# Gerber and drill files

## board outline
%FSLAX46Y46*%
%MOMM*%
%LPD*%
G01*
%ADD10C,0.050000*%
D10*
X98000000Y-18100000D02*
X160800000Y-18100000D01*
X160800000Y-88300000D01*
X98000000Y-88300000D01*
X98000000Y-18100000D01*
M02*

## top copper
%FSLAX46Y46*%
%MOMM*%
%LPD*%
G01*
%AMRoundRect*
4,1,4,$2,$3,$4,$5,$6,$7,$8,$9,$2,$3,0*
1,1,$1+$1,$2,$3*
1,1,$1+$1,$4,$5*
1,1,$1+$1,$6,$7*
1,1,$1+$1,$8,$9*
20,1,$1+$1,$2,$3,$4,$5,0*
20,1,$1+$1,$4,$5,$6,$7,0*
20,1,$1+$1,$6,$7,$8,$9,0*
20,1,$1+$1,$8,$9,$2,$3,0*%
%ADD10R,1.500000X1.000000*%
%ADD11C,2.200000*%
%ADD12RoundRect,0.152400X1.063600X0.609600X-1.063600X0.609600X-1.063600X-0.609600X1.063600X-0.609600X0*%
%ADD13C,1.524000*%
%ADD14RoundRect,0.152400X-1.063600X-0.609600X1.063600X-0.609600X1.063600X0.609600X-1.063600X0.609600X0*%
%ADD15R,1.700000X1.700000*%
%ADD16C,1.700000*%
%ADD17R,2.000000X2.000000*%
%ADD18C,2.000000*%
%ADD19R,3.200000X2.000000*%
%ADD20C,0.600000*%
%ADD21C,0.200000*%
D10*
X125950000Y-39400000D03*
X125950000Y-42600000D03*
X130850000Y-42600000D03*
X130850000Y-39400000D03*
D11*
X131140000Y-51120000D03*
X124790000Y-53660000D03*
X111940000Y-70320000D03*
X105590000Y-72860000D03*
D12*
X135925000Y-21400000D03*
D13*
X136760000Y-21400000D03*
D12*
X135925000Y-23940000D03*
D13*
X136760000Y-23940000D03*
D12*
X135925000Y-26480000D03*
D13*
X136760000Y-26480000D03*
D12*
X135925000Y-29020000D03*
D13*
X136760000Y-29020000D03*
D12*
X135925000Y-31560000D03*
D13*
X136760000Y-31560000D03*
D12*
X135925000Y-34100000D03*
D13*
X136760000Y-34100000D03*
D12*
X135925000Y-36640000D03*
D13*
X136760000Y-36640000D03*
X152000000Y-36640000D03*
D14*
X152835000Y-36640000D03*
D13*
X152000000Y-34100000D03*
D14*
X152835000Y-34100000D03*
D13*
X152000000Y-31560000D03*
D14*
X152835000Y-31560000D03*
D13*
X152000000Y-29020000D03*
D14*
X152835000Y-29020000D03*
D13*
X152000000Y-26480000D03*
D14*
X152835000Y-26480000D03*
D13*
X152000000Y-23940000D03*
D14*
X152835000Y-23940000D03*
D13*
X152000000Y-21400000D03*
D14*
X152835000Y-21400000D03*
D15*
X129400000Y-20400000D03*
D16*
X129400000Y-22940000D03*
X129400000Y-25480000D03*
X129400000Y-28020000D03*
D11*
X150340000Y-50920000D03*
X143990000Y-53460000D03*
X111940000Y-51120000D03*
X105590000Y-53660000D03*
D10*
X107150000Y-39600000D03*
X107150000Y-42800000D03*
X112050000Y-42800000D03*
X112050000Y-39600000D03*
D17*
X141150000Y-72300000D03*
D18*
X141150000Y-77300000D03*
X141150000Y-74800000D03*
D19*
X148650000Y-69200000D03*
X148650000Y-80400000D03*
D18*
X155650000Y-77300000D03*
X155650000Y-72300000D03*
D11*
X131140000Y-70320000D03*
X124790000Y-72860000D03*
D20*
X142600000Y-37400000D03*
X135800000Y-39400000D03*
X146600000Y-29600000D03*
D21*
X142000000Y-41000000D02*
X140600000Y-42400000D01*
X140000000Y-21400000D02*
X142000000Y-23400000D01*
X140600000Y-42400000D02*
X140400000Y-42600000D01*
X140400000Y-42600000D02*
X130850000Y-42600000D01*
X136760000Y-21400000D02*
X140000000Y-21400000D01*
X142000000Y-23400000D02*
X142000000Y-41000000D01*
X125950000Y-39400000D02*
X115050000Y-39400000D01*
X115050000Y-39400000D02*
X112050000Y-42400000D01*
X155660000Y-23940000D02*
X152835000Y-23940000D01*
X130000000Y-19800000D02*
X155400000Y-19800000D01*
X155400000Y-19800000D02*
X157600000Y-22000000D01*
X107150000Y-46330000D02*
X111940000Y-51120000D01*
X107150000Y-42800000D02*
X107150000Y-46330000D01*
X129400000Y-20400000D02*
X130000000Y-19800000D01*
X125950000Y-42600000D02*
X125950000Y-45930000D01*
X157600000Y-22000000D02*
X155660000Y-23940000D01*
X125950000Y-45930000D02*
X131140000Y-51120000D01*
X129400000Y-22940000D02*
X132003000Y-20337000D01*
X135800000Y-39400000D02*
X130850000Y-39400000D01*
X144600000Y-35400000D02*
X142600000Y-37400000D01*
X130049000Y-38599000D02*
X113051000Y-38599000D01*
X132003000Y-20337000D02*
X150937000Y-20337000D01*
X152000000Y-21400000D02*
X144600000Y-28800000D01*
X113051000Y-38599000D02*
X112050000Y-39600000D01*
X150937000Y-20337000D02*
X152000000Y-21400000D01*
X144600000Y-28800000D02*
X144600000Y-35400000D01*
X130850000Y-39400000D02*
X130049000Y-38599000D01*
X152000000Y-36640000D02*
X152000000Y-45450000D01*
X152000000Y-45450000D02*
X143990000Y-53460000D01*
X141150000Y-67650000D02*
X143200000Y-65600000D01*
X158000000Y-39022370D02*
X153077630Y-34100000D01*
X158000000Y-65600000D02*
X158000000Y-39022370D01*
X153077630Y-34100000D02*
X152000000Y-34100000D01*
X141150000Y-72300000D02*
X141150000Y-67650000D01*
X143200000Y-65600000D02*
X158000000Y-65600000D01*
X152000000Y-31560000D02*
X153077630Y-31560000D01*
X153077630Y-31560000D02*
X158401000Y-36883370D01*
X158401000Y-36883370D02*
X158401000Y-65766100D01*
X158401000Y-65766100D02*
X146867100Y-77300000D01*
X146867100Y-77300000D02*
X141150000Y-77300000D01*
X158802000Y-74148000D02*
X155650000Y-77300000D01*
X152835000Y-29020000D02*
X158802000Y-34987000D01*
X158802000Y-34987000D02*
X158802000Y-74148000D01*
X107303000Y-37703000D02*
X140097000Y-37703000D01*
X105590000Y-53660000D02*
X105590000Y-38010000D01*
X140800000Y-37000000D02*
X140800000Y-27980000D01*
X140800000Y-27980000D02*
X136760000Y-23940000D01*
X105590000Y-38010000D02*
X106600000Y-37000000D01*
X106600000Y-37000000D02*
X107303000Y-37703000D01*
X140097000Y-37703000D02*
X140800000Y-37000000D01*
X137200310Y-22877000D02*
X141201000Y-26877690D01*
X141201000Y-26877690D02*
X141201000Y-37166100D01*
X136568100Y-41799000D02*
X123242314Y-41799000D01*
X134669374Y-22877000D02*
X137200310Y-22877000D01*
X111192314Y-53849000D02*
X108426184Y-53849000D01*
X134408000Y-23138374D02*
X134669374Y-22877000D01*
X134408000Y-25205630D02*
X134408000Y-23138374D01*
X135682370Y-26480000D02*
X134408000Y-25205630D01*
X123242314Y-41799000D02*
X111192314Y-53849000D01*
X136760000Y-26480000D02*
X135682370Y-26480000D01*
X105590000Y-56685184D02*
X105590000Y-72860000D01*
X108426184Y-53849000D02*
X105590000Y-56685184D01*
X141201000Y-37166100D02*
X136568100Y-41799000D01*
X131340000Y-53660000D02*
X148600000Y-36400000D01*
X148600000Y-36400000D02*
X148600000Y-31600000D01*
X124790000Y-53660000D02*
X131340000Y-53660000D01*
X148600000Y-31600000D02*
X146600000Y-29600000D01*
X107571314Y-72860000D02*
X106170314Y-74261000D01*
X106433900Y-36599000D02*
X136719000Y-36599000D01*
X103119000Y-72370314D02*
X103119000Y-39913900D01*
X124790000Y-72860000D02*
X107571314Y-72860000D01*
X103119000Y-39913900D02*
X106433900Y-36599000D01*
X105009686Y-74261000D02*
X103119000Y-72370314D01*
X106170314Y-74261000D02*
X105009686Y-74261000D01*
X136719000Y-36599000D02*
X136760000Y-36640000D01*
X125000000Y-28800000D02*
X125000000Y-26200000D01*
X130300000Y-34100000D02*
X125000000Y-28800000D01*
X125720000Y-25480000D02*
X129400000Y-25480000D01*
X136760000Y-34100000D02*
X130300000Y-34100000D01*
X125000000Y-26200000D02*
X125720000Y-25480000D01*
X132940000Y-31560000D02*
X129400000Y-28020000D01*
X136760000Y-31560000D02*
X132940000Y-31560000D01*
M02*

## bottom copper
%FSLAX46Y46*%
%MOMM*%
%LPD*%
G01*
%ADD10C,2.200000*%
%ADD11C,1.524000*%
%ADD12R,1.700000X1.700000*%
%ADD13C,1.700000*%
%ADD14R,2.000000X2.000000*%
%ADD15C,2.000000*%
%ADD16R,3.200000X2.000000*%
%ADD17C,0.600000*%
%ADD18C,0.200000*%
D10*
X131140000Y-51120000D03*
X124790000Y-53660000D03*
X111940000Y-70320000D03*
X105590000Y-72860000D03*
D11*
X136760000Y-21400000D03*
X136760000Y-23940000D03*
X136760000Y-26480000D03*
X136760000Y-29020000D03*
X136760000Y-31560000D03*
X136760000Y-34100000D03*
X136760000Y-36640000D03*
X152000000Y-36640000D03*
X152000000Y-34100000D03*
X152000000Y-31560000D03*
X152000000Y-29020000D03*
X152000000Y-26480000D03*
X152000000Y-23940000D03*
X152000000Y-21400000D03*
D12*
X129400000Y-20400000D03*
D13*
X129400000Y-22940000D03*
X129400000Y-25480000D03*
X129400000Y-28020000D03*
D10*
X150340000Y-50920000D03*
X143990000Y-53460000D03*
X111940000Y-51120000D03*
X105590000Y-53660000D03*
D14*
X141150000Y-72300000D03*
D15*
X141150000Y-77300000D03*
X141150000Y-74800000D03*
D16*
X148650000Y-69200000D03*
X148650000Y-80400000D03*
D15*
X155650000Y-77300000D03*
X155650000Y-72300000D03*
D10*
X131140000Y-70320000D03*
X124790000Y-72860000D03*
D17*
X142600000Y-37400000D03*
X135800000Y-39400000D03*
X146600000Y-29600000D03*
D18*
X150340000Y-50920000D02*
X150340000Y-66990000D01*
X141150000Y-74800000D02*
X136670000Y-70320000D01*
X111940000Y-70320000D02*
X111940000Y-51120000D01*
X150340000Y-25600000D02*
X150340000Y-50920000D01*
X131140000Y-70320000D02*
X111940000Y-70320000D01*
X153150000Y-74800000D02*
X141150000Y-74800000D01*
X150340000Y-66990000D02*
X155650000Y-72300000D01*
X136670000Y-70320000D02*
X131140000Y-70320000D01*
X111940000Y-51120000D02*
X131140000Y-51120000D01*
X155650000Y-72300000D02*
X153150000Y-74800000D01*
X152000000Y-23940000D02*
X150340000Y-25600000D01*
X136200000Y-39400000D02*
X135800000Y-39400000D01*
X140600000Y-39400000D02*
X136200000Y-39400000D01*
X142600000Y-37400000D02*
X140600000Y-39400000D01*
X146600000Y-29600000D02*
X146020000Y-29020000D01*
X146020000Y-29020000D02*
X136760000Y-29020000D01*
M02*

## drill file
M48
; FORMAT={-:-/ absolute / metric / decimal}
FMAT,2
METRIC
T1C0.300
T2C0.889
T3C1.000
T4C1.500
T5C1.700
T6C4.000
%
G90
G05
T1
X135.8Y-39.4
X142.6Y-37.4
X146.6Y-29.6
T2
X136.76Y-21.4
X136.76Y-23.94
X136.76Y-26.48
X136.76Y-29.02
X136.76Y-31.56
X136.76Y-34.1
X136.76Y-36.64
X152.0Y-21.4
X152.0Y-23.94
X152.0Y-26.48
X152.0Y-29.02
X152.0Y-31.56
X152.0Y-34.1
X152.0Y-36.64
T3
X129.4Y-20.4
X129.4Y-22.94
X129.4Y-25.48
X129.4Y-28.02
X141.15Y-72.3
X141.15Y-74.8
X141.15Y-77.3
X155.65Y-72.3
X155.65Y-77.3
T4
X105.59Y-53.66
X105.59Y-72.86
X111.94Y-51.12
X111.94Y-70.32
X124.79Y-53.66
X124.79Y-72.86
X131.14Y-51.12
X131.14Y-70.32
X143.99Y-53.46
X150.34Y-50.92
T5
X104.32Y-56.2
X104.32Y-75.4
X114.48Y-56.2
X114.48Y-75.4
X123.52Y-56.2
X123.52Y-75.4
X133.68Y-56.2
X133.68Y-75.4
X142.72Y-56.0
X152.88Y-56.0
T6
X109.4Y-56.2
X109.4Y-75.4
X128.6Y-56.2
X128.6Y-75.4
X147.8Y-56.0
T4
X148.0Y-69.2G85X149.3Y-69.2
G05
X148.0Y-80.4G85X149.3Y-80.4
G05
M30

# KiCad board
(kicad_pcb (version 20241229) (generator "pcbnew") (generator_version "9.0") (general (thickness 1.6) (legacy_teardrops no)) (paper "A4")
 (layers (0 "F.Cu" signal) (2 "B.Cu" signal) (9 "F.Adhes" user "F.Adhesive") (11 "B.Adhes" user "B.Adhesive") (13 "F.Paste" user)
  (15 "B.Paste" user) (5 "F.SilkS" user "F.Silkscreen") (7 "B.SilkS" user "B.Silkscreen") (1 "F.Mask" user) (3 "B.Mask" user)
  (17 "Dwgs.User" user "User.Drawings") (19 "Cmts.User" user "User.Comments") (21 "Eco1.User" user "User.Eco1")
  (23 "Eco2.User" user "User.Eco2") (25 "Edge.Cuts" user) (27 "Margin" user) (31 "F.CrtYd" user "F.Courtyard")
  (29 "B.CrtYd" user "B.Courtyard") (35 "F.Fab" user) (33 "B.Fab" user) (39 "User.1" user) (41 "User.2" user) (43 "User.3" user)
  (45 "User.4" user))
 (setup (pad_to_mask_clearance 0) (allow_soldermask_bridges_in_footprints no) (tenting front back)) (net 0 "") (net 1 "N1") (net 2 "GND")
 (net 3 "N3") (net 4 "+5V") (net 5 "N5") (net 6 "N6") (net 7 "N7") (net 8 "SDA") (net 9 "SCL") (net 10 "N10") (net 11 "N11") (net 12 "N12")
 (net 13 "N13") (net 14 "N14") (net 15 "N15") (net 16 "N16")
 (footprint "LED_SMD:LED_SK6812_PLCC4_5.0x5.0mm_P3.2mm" (layer "F.Cu") (at 128.4 41)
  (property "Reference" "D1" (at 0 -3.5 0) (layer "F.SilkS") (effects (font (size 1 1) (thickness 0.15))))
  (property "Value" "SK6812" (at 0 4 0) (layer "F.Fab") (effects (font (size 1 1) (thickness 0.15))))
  (pad "1" smd rect (at -2.45 -1.6 180) (size 1.5 1) (layers "F.Cu" "F.Mask" "F.Paste") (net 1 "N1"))
  (pad "2" smd rect (at -2.45 1.6 180) (size 1.5 1) (layers "F.Cu" "F.Mask" "F.Paste") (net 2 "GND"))
  (pad "3" smd rect (at 2.45 1.6 180) (size 1.5 1) (layers "F.Cu" "F.Mask" "F.Paste") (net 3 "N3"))
  (pad "4" smd rect (at 2.45 -1.6 180) (size 1.5 1) (layers "F.Cu" "F.Mask" "F.Paste") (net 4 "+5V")))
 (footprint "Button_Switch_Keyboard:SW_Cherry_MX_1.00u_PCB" (layer "F.Cu") (at 131.14 51.12)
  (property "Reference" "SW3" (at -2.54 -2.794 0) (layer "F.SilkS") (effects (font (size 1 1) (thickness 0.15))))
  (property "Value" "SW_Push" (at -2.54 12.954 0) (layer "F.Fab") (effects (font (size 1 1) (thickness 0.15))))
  (pad "" np_thru_hole circle (at -7.62 5.08) (size 1.7 1.7) (drill 1.7) (layers "*.Cu" "*.Mask"))
  (pad "" np_thru_hole circle (at -2.54 5.08) (size 4 4) (drill 4) (layers "*.Cu" "*.Mask"))
  (pad "" np_thru_hole circle (at 2.54 5.08) (size 1.7 1.7) (drill 1.7) (layers "*.Cu" "*.Mask"))
  (pad "1" thru_hole circle (at 0 0) (size 2.2 2.2) (drill 1.5) (layers "*.Cu" "*.Mask") (remove_unused_layers no) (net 2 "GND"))
  (pad "2" thru_hole circle (at -6.35 2.54) (size 2.2 2.2) (drill 1.5) (layers "*.Cu" "*.Mask") (remove_unused_layers no) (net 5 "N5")))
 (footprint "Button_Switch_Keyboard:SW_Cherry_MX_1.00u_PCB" (layer "F.Cu") (at 111.94 70.32)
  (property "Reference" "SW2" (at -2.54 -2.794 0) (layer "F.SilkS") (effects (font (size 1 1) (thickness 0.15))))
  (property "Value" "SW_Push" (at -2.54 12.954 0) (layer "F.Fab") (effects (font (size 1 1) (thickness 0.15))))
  (pad "" np_thru_hole circle (at -7.62 5.08) (size 1.7 1.7) (drill 1.7) (layers "*.Cu" "*.Mask"))
  (pad "" np_thru_hole circle (at -2.54 5.08) (size 4 4) (drill 4) (layers "*.Cu" "*.Mask"))
  (pad "" np_thru_hole circle (at 2.54 5.08) (size 1.7 1.7) (drill 1.7) (layers "*.Cu" "*.Mask"))
  (pad "1" thru_hole circle (at 0 0) (size 2.2 2.2) (drill 1.5) (layers "*.Cu" "*.Mask") (remove_unused_layers no) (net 2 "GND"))
  (pad "2" thru_hole circle (at -6.35 2.54) (size 2.2 2.2) (drill 1.5) (layers "*.Cu" "*.Mask") (remove_unused_layers no) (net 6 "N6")))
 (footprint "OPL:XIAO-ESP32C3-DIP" (layer "F.Cu") (at 144.5 29.02)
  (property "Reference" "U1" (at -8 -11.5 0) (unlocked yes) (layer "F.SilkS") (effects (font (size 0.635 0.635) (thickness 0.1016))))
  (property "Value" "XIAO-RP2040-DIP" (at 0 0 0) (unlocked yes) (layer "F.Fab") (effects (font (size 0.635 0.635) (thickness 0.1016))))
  (pad "1" smd roundrect (at -8.575 -7.62 180) (size 2.432 1.524) (layers "F.Cu" "F.Mask") (roundrect_rratio 0.1) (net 3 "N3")
   (thermal_bridge_angle 45))
  (pad "1" thru_hole circle (at -7.74 -7.62 180) (size 1.524 1.524) (drill 0.889) (layers "*.Cu" "*.Mask") (remove_unused_layers no)
   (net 3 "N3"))
  (pad "2" smd roundrect (at -8.575 -5.08 180) (size 2.432 1.524) (layers "F.Cu" "F.Mask") (roundrect_rratio 0.1) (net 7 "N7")
   (thermal_bridge_angle 45))
  (pad "2" thru_hole circle (at -7.74 -5.08 180) (size 1.524 1.524) (drill 0.889) (layers "*.Cu" "*.Mask") (remove_unused_layers no)
   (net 7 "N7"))
  (pad "3" smd roundrect (at -8.575 -2.54 180) (size 2.432 1.524) (layers "F.Cu" "F.Mask") (roundrect_rratio 0.1) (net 6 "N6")
   (thermal_bridge_angle 45))
  (pad "3" thru_hole circle (at -7.74 -2.54 180) (size 1.524 1.524) (drill 0.889) (layers "*.Cu" "*.Mask") (remove_unused_layers no)
   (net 6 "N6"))
  (pad "4" smd roundrect (at -8.575 0 180) (size 2.432 1.524) (layers "F.Cu" "F.Mask") (roundrect_rratio 0.1) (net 5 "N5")
   (thermal_bridge_angle 45))
  (pad "4" thru_hole circle (at -7.74 0 180) (size 1.524 1.524) (drill 0.889) (layers "*.Cu" "*.Mask") (remove_unused_layers no)
   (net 5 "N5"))
  (pad "5" smd roundrect (at -8.575 2.54 180) (size 2.432 1.524) (layers "F.Cu" "F.Mask") (roundrect_rratio 0.1) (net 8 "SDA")
   (thermal_bridge_angle 45))
  (pad "5" thru_hole circle (at -7.74 2.54 180) (size 1.524 1.524) (drill 0.889) (layers "*.Cu" "*.Mask") (remove_unused_layers no)
   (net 8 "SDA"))
  (pad "6" smd roundrect (at -8.575 5.08 180) (size 2.432 1.524) (layers "F.Cu" "F.Mask") (roundrect_rratio 0.1) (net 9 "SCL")
   (thermal_bridge_angle 45))
  (pad "6" thru_hole circle (at -7.74 5.08 180) (size 1.524 1.524) (drill 0.889) (layers "*.Cu" "*.Mask") (remove_unused_layers no)
   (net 9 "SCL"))
  (pad "7" smd roundrect (at -8.575 7.62 180) (size 2.432 1.524) (layers "F.Cu" "F.Mask") (roundrect_rratio 0.1) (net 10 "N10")
   (thermal_bridge_angle 45))
  (pad "7" thru_hole circle (at -7.74 7.62 180) (size 1.524 1.524) (drill 0.889) (layers "*.Cu" "*.Mask") (remove_unused_layers no)
   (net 10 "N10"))
  (pad "8" thru_hole circle (at 7.5 7.62) (size 1.524 1.524) (drill 0.889) (layers "*.Cu" "*.Mask") (remove_unused_layers no) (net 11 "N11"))
  (pad "8" smd roundrect (at 8.335 7.62) (size 2.432 1.524) (layers "F.Cu" "F.Mask") (roundrect_rratio 0.1) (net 11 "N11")
   (thermal_bridge_angle 45))
  (pad "9" thru_hole circle (at 7.5 5.08) (size 1.524 1.524) (drill 0.889) (layers "*.Cu" "*.Mask") (remove_unused_layers no) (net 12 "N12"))
  (pad "9" smd roundrect (at 8.335 5.08) (size 2.432 1.524) (layers "F.Cu" "F.Mask") (roundrect_rratio 0.1) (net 12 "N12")
   (thermal_bridge_angle 45))
  (pad "10" thru_hole circle (at 7.5 2.54) (size 1.524 1.524) (drill 0.889) (layers "*.Cu" "*.Mask") (remove_unused_layers no)
   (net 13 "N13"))
  (pad "10" smd roundrect (at 8.335 2.54) (size 2.432 1.524) (layers "F.Cu" "F.Mask") (roundrect_rratio 0.1) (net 13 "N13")
   (thermal_bridge_angle 45))
  (pad "11" thru_hole circle (at 7.5 0) (size 1.524 1.524) (drill 0.889) (layers "*.Cu" "*.Mask") (remove_unused_layers no) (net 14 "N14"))
  (pad "11" smd roundrect (at 8.335 0) (size 2.432 1.524) (layers "F.Cu" "F.Mask") (roundrect_rratio 0.1) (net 14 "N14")
   (thermal_bridge_angle 45))
  (pad "12" thru_hole circle (at 7.5 -2.54) (size 1.524 1.524) (drill 0.889) (layers "*.Cu" "*.Mask") (remove_unused_layers no)
   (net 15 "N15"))
  (pad "12" smd roundrect (at 8.335 -2.54) (size 2.432 1.524) (layers "F.Cu" "F.Mask") (roundrect_rratio 0.1) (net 15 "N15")
   (thermal_bridge_angle 45))
  (pad "13" thru_hole circle (at 7.5 -5.08) (size 1.524 1.524) (drill 0.889) (layers "*.Cu" "*.Mask") (remove_unused_layers no)
   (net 2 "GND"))
  (pad "13" smd roundrect (at 8.335 -5.08) (size 2.432 1.524) (layers "F.Cu" "F.Mask") (roundrect_rratio 0.1) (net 2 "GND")
   (thermal_bridge_angle 45))
  (pad "14" thru_hole circle (at 7.5 -7.62) (size 1.524 1.524) (drill 0.889) (layers "*.Cu" "*.Mask") (remove_unused_layers no)
   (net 4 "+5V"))
  (pad "14" smd roundrect (at 8.335 -7.62) (size 2.432 1.524) (layers "F.Cu" "F.Mask") (roundrect_rratio 0.1) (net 4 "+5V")
   (thermal_bridge_angle 45)))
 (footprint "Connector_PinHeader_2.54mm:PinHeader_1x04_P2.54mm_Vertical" (layer "F.Cu") (at 129.4 20.4)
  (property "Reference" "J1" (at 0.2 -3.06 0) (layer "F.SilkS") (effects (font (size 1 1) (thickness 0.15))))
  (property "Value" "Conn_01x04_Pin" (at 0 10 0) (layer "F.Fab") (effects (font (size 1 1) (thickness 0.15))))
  (pad "1" thru_hole rect (at 0 0) (size 1.7 1.7) (drill 1) (layers "*.Cu" "*.Mask") (remove_unused_layers no) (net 2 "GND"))
  (pad "2" thru_hole circle (at 0 2.54) (size 1.7 1.7) (drill 1) (layers "*.Cu" "*.Mask") (remove_unused_layers no) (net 4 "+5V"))
  (pad "3" thru_hole circle (at 0 5.08) (size 1.7 1.7) (drill 1) (layers "*.Cu" "*.Mask") (remove_unused_layers no) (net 9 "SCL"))
  (pad "4" thru_hole circle (at 0 7.62) (size 1.7 1.7) (drill 1) (layers "*.Cu" "*.Mask") (remove_unused_layers no) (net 8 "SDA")))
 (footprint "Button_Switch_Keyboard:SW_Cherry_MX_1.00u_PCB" (layer "F.Cu") (at 150.34 50.92)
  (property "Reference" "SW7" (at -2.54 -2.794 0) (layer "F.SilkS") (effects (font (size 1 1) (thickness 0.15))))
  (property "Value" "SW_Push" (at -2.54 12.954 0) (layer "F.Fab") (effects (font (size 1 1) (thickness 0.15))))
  (pad "" np_thru_hole circle (at -7.62 5.08) (size 1.7 1.7) (drill 1.7) (layers "*.Cu" "*.Mask"))
  (pad "" np_thru_hole circle (at -2.54 5.08) (size 4 4) (drill 4) (layers "*.Cu" "*.Mask"))
  (pad "" np_thru_hole circle (at 2.54 5.08) (size 1.7 1.7) (drill 1.7) (layers "*.Cu" "*.Mask"))
  (pad "1" thru_hole circle (at 0 0) (size 2.2 2.2) (drill 1.5) (layers "*.Cu" "*.Mask") (remove_unused_layers no) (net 2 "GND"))
  (pad "2" thru_hole circle (at -6.35 2.54) (size 2.2 2.2) (drill 1.5) (layers "*.Cu" "*.Mask") (remove_unused_layers no) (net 11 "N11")))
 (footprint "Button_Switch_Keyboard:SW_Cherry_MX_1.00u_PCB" (layer "F.Cu") (at 111.94 51.12)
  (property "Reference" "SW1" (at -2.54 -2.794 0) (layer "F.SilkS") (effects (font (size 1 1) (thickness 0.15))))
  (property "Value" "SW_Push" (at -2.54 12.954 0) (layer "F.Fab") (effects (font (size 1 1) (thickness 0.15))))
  (pad "" np_thru_hole circle (at -7.62 5.08) (size 1.7 1.7) (drill 1.7) (layers "*.Cu" "*.Mask"))
  (pad "" np_thru_hole circle (at -2.54 5.08) (size 4 4) (drill 4) (layers "*.Cu" "*.Mask"))
  (pad "" np_thru_hole circle (at 2.54 5.08) (size 1.7 1.7) (drill 1.7) (layers "*.Cu" "*.Mask"))
  (pad "1" thru_hole circle (at 0 0) (size 2.2 2.2) (drill 1.5) (layers "*.Cu" "*.Mask") (remove_unused_layers no) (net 2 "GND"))
  (pad "2" thru_hole circle (at -6.35 2.54) (size 2.2 2.2) (drill 1.5) (layers "*.Cu" "*.Mask") (remove_unused_layers no) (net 7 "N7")))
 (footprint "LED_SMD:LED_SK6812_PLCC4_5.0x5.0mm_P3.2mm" (layer "F.Cu") (at 109.6 41.2)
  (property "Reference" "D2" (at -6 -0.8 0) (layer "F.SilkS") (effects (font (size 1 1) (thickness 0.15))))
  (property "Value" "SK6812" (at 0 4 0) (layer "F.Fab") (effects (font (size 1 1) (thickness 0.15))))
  (pad "1" smd rect (at -2.45 -1.6 180) (size 1.5 1) (layers "F.Cu" "F.Mask" "F.Paste") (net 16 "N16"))
  (pad "2" smd rect (at -2.45 1.6 180) (size 1.5 1) (layers "F.Cu" "F.Mask" "F.Paste") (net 2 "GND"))
  (pad "3" smd rect (at 2.45 1.6 180) (size 1.5 1) (layers "F.Cu" "F.Mask" "F.Paste") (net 1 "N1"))
  (pad "4" smd rect (at 2.45 -1.6 180) (size 1.5 1) (layers "F.Cu" "F.Mask" "F.Paste") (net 4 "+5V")))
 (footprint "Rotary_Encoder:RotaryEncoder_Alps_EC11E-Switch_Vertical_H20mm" (layer "F.Cu") (at 141.15 72.3)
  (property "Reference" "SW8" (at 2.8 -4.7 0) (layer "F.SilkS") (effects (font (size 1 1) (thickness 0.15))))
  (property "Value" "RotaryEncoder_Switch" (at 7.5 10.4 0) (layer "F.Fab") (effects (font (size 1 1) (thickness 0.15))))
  (pad "A" thru_hole rect (at 0 0) (size 2 2) (drill 1) (layers "*.Cu" "*.Mask") (remove_unused_layers no) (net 12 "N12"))
  (pad "B" thru_hole circle (at 0 5) (size 2 2) (drill 1) (layers "*.Cu" "*.Mask") (remove_unused_layers no) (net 13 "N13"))
  (pad "C" thru_hole circle (at 0 2.5) (size 2 2) (drill 1) (layers "*.Cu" "*.Mask") (remove_unused_layers no) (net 2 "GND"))
  (pad "MP" thru_hole rect (at 7.5 -3.1) (size 3.2 2) (drill oval 2.8 1.5) (layers "*.Cu" "*.Mask") (remove_unused_layers no))
  (pad "MP" thru_hole rect (at 7.5 8.1) (size 3.2 2) (drill oval 2.8 1.5) (layers "*.Cu" "*.Mask") (remove_unused_layers no))
  (pad "S1" thru_hole circle (at 14.5 5) (size 2 2) (drill 1) (layers "*.Cu" "*.Mask") (remove_unused_layers no) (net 14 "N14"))
  (pad "S2" thru_hole circle (at 14.5 0) (size 2 2) (drill 1) (layers "*.Cu" "*.Mask") (remove_unused_layers no) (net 2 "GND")))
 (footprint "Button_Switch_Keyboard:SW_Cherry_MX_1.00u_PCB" (layer "F.Cu") (at 131.14 70.32)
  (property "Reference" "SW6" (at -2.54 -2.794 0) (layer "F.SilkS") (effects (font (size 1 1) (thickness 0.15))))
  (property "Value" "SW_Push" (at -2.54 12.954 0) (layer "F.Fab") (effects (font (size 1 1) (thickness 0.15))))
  (pad "" np_thru_hole circle (at -7.62 5.08) (size 1.7 1.7) (drill 1.7) (layers "*.Cu" "*.Mask"))
  (pad "" np_thru_hole circle (at -2.54 5.08) (size 4 4) (drill 4) (layers "*.Cu" "*.Mask"))
  (pad "" np_thru_hole circle (at 2.54 5.08) (size 1.7 1.7) (drill 1.7) (layers "*.Cu" "*.Mask"))
  (pad "1" thru_hole circle (at 0 0) (size 2.2 2.2) (drill 1.5) (layers "*.Cu" "*.Mask") (remove_unused_layers no) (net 2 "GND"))
  (pad "2" thru_hole circle (at -6.35 2.54) (size 2.2 2.2) (drill 1.5) (layers "*.Cu" "*.Mask") (remove_unused_layers no) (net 10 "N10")))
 (gr_rect (start 98 18.1) (end 160.8 88.3) (stroke (width 0.05) (type default)) (fill no) (layer "Edge.Cuts"))
 (segment (start 142 41) (end 140.6 42.4) (width 0.2) (layer "F.Cu") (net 3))
 (segment (start 140 21.4) (end 142 23.4) (width 0.2) (layer "F.Cu") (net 3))
 (segment (start 140.6 42.4) (end 140.4 42.6) (width 0.2) (layer "F.Cu") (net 3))
 (segment (start 140.4 42.6) (end 130.85 42.6) (width 0.2) (layer "F.Cu") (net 3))
 (segment (start 136.76 21.4) (end 140 21.4) (width 0.2) (layer "F.Cu") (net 3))
 (segment (start 142 23.4) (end 142 41) (width 0.2) (layer "F.Cu") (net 3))
 (segment (start 125.95 39.4) (end 115.05 39.4) (width 0.2) (layer "F.Cu") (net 1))
 (segment (start 115.05 39.4) (end 112.05 42.4) (width 0.2) (layer "F.Cu") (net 1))
 (segment (start 155.66 23.94) (end 152.835 23.94) (width 0.2) (layer "F.Cu") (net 2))
 (segment (start 130 19.8) (end 155.4 19.8) (width 0.2) (layer "F.Cu") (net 2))
 (segment (start 155.4 19.8) (end 157.6 22) (width 0.2) (layer "F.Cu") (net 2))
 (segment (start 107.15 46.33) (end 111.94 51.12) (width 0.2) (layer "F.Cu") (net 2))
 (segment (start 107.15 42.8) (end 107.15 46.33) (width 0.2) (layer "F.Cu") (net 2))
 (segment (start 129.4 20.4) (end 130 19.8) (width 0.2) (layer "F.Cu") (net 2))
 (segment (start 125.95 42.6) (end 125.95 45.93) (width 0.2) (layer "F.Cu") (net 2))
 (segment (start 157.6 22) (end 155.66 23.94) (width 0.2) (layer "F.Cu") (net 2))
 (segment (start 125.95 45.93) (end 131.14 51.12) (width 0.2) (layer "F.Cu") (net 2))
 (segment (start 150.34 50.92) (end 150.34 66.99) (width 0.2) (layer "B.Cu") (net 2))
 (segment (start 141.15 74.8) (end 136.67 70.32) (width 0.2) (layer "B.Cu") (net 2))
 (segment (start 111.94 70.32) (end 111.94 51.12) (width 0.2) (layer "B.Cu") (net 2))
 (segment (start 150.34 25.6) (end 150.34 50.92) (width 0.2) (layer "B.Cu") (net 2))
 (segment (start 131.14 70.32) (end 111.94 70.32) (width 0.2) (layer "B.Cu") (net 2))
 (segment (start 153.15 74.8) (end 141.15 74.8) (width 0.2) (layer "B.Cu") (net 2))
 (segment (start 150.34 66.99) (end 155.65 72.3) (width 0.2) (layer "B.Cu") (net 2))
 (segment (start 136.67 70.32) (end 131.14 70.32) (width 0.2) (layer "B.Cu") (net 2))
 (segment (start 111.94 51.12) (end 131.14 51.12) (width 0.2) (layer "B.Cu") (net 2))
 (segment (start 155.65 72.3) (end 153.15 74.8) (width 0.2) (layer "B.Cu") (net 2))
 (segment (start 152 23.94) (end 150.34 25.6) (width 0.2) (layer "B.Cu") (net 2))
 (segment (start 129.4 22.94) (end 132.003 20.337) (width 0.2) (layer "F.Cu") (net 4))
 (segment (start 135.8 39.4) (end 130.85 39.4) (width 0.2) (layer "F.Cu") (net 4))
 (segment (start 144.6 35.4) (end 142.6 37.4) (width 0.2) (layer "F.Cu") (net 4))
 (segment (start 130.049 38.599) (end 113.051 38.599) (width 0.2) (layer "F.Cu") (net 4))
 (segment (start 132.003 20.337) (end 150.937 20.337) (width 0.2) (layer "F.Cu") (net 4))
 (segment (start 152 21.4) (end 144.6 28.8) (width 0.2) (layer "F.Cu") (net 4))
 (segment (start 113.051 38.599) (end 112.05 39.6) (width 0.2) (layer "F.Cu") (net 4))
 (segment (start 150.937 20.337) (end 152 21.4) (width 0.2) (layer "F.Cu") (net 4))
 (segment (start 144.6 28.8) (end 144.6 35.4) (width 0.2) (layer "F.Cu") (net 4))
 (segment (start 130.85 39.4) (end 130.049 38.599) (width 0.2) (layer "F.Cu") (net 4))
 (via (at 142.6 37.4) (size 0.6) (drill 0.3) (layers "F.Cu" "B.Cu") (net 4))
 (via (at 135.8 39.4) (size 0.6) (drill 0.3) (layers "F.Cu" "B.Cu") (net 4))
 (segment (start 136.2 39.4) (end 135.8 39.4) (width 0.2) (layer "B.Cu") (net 4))
 (segment (start 140.6 39.4) (end 136.2 39.4) (width 0.2) (layer "B.Cu") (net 4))
 (segment (start 142.6 37.4) (end 140.6 39.4) (width 0.2) (layer "B.Cu") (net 4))
 (segment (start 152 36.64) (end 152 45.45) (width 0.2) (layer "F.Cu") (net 11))
 (segment (start 152 45.45) (end 143.99 53.46) (width 0.2) (layer "F.Cu") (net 11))
 (segment (start 141.15 67.65) (end 143.2 65.6) (width 0.2) (layer "F.Cu") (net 12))
 (segment (start 158 39.02237) (end 153.07763 34.1) (width 0.2) (layer "F.Cu") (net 12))
 (segment (start 158 65.6) (end 158 39.02237) (width 0.2) (layer "F.Cu") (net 12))
 (segment (start 153.07763 34.1) (end 152 34.1) (width 0.2) (layer "F.Cu") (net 12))
 (segment (start 141.15 72.3) (end 141.15 67.65) (width 0.2) (layer "F.Cu") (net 12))
 (segment (start 143.2 65.6) (end 158 65.6) (width 0.2) (layer "F.Cu") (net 12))
 (segment (start 152 31.56) (end 153.07763 31.56) (width 0.2) (layer "F.Cu") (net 13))
 (segment (start 153.07763 31.56) (end 158.401 36.88337) (width 0.2) (layer "F.Cu") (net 13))
 (segment (start 158.401 36.88337) (end 158.401 65.7661) (width 0.2) (layer "F.Cu") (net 13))
 (segment (start 158.401 65.7661) (end 146.8671 77.3) (width 0.2) (layer "F.Cu") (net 13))
 (segment (start 146.8671 77.3) (end 141.15 77.3) (width 0.2) (layer "F.Cu") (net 13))
 (segment (start 158.802 74.148) (end 155.65 77.3) (width 0.2) (layer "F.Cu") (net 14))
 (segment (start 152.835 29.02) (end 158.802 34.987) (width 0.2) (layer "F.Cu") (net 14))
 (segment (start 158.802 34.987) (end 158.802 74.148) (width 0.2) (layer "F.Cu") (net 14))
 (segment (start 107.303 37.703) (end 140.097 37.703) (width 0.2) (layer "F.Cu") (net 7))
 (segment (start 105.59 53.66) (end 105.59 38.01) (width 0.2) (layer "F.Cu") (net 7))
 (segment (start 140.8 37) (end 140.8 27.98) (width 0.2) (layer "F.Cu") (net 7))
 (segment (start 140.8 27.98) (end 136.76 23.94) (width 0.2) (layer "F.Cu") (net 7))
 (segment (start 105.59 38.01) (end 106.6 37) (width 0.2) (layer "F.Cu") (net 7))
 (segment (start 106.6 37) (end 107.303 37.703) (width 0.2) (layer "F.Cu") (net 7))
 (segment (start 140.097 37.703) (end 140.8 37) (width 0.2) (layer "F.Cu") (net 7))
 (segment (start 137.20031 22.877) (end 141.201 26.87769) (width 0.2) (layer "F.Cu") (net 6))
 (segment (start 141.201 26.87769) (end 141.201 37.1661) (width 0.2) (layer "F.Cu") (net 6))
 (segment (start 136.5681 41.799) (end 123.242314 41.799) (width 0.2) (layer "F.Cu") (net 6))
 (segment (start 134.669374 22.877) (end 137.20031 22.877) (width 0.2) (layer "F.Cu") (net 6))
 (segment (start 111.192314 53.849) (end 108.426184 53.849) (width 0.2) (layer "F.Cu") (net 6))
 (segment (start 134.408 23.138374) (end 134.669374 22.877) (width 0.2) (layer "F.Cu") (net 6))
 (segment (start 134.408 25.20563) (end 134.408 23.138374) (width 0.2) (layer "F.Cu") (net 6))
 (segment (start 135.68237 26.48) (end 134.408 25.20563) (width 0.2) (layer "F.Cu") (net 6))
 (segment (start 123.242314 41.799) (end 111.192314 53.849) (width 0.2) (layer "F.Cu") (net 6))
 (segment (start 136.76 26.48) (end 135.68237 26.48) (width 0.2) (layer "F.Cu") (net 6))
 (segment (start 105.59 56.685184) (end 105.59 72.86) (width 0.2) (layer "F.Cu") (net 6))
 (segment (start 108.426184 53.849) (end 105.59 56.685184) (width 0.2) (layer "F.Cu") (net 6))
 (segment (start 141.201 37.1661) (end 136.5681 41.799) (width 0.2) (layer "F.Cu") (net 6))
 (segment (start 131.34 53.66) (end 148.6 36.4) (width 0.2) (layer "F.Cu") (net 5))
 (segment (start 148.6 36.4) (end 148.6 31.6) (width 0.2) (layer "F.Cu") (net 5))
 (segment (start 124.79 53.66) (end 131.34 53.66) (width 0.2) (layer "F.Cu") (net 5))
 (segment (start 148.6 31.6) (end 146.6 29.6) (width 0.2) (layer "F.Cu") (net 5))
 (via (at 146.6 29.6) (size 0.6) (drill 0.3) (layers "F.Cu" "B.Cu") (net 5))
 (segment (start 146.6 29.6) (end 146.02 29.02) (width 0.2) (layer "B.Cu") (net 5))
 (segment (start 146.02 29.02) (end 136.76 29.02) (width 0.2) (layer "B.Cu") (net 5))
 (segment (start 107.571314 72.86) (end 106.170314 74.261) (width 0.2) (layer "F.Cu") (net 10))
 (segment (start 106.4339 36.599) (end 136.719 36.599) (width 0.2) (layer "F.Cu") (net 10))
 (segment (start 103.119 72.370314) (end 103.119 39.9139) (width 0.2) (layer "F.Cu") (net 10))
 (segment (start 124.79 72.86) (end 107.571314 72.86) (width 0.2) (layer "F.Cu") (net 10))
 (segment (start 103.119 39.9139) (end 106.4339 36.599) (width 0.2) (layer "F.Cu") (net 10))
 (segment (start 105.009686 74.261) (end 103.119 72.370314) (width 0.2) (layer "F.Cu") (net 10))
 (segment (start 106.170314 74.261) (end 105.009686 74.261) (width 0.2) (layer "F.Cu") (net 10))
 (segment (start 136.719 36.599) (end 136.76 36.64) (width 0.2) (layer "F.Cu") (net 10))
 (segment (start 125 28.8) (end 125 26.2) (width 0.2) (layer "F.Cu") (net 9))
 (segment (start 130.3 34.1) (end 125 28.8) (width 0.2) (layer "F.Cu") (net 9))
 (segment (start 125.72 25.48) (end 129.4 25.48) (width 0.2) (layer "F.Cu") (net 9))
 (segment (start 136.76 34.1) (end 130.3 34.1) (width 0.2) (layer "F.Cu") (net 9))
 (segment (start 125 26.2) (end 125.72 25.48) (width 0.2) (layer "F.Cu") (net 9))
 (segment (start 132.94 31.56) (end 129.4 28.02) (width 0.2) (layer "F.Cu") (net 8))
 (segment (start 136.76 31.56) (end 132.94 31.56) (width 0.2) (layer "F.Cu") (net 8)))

